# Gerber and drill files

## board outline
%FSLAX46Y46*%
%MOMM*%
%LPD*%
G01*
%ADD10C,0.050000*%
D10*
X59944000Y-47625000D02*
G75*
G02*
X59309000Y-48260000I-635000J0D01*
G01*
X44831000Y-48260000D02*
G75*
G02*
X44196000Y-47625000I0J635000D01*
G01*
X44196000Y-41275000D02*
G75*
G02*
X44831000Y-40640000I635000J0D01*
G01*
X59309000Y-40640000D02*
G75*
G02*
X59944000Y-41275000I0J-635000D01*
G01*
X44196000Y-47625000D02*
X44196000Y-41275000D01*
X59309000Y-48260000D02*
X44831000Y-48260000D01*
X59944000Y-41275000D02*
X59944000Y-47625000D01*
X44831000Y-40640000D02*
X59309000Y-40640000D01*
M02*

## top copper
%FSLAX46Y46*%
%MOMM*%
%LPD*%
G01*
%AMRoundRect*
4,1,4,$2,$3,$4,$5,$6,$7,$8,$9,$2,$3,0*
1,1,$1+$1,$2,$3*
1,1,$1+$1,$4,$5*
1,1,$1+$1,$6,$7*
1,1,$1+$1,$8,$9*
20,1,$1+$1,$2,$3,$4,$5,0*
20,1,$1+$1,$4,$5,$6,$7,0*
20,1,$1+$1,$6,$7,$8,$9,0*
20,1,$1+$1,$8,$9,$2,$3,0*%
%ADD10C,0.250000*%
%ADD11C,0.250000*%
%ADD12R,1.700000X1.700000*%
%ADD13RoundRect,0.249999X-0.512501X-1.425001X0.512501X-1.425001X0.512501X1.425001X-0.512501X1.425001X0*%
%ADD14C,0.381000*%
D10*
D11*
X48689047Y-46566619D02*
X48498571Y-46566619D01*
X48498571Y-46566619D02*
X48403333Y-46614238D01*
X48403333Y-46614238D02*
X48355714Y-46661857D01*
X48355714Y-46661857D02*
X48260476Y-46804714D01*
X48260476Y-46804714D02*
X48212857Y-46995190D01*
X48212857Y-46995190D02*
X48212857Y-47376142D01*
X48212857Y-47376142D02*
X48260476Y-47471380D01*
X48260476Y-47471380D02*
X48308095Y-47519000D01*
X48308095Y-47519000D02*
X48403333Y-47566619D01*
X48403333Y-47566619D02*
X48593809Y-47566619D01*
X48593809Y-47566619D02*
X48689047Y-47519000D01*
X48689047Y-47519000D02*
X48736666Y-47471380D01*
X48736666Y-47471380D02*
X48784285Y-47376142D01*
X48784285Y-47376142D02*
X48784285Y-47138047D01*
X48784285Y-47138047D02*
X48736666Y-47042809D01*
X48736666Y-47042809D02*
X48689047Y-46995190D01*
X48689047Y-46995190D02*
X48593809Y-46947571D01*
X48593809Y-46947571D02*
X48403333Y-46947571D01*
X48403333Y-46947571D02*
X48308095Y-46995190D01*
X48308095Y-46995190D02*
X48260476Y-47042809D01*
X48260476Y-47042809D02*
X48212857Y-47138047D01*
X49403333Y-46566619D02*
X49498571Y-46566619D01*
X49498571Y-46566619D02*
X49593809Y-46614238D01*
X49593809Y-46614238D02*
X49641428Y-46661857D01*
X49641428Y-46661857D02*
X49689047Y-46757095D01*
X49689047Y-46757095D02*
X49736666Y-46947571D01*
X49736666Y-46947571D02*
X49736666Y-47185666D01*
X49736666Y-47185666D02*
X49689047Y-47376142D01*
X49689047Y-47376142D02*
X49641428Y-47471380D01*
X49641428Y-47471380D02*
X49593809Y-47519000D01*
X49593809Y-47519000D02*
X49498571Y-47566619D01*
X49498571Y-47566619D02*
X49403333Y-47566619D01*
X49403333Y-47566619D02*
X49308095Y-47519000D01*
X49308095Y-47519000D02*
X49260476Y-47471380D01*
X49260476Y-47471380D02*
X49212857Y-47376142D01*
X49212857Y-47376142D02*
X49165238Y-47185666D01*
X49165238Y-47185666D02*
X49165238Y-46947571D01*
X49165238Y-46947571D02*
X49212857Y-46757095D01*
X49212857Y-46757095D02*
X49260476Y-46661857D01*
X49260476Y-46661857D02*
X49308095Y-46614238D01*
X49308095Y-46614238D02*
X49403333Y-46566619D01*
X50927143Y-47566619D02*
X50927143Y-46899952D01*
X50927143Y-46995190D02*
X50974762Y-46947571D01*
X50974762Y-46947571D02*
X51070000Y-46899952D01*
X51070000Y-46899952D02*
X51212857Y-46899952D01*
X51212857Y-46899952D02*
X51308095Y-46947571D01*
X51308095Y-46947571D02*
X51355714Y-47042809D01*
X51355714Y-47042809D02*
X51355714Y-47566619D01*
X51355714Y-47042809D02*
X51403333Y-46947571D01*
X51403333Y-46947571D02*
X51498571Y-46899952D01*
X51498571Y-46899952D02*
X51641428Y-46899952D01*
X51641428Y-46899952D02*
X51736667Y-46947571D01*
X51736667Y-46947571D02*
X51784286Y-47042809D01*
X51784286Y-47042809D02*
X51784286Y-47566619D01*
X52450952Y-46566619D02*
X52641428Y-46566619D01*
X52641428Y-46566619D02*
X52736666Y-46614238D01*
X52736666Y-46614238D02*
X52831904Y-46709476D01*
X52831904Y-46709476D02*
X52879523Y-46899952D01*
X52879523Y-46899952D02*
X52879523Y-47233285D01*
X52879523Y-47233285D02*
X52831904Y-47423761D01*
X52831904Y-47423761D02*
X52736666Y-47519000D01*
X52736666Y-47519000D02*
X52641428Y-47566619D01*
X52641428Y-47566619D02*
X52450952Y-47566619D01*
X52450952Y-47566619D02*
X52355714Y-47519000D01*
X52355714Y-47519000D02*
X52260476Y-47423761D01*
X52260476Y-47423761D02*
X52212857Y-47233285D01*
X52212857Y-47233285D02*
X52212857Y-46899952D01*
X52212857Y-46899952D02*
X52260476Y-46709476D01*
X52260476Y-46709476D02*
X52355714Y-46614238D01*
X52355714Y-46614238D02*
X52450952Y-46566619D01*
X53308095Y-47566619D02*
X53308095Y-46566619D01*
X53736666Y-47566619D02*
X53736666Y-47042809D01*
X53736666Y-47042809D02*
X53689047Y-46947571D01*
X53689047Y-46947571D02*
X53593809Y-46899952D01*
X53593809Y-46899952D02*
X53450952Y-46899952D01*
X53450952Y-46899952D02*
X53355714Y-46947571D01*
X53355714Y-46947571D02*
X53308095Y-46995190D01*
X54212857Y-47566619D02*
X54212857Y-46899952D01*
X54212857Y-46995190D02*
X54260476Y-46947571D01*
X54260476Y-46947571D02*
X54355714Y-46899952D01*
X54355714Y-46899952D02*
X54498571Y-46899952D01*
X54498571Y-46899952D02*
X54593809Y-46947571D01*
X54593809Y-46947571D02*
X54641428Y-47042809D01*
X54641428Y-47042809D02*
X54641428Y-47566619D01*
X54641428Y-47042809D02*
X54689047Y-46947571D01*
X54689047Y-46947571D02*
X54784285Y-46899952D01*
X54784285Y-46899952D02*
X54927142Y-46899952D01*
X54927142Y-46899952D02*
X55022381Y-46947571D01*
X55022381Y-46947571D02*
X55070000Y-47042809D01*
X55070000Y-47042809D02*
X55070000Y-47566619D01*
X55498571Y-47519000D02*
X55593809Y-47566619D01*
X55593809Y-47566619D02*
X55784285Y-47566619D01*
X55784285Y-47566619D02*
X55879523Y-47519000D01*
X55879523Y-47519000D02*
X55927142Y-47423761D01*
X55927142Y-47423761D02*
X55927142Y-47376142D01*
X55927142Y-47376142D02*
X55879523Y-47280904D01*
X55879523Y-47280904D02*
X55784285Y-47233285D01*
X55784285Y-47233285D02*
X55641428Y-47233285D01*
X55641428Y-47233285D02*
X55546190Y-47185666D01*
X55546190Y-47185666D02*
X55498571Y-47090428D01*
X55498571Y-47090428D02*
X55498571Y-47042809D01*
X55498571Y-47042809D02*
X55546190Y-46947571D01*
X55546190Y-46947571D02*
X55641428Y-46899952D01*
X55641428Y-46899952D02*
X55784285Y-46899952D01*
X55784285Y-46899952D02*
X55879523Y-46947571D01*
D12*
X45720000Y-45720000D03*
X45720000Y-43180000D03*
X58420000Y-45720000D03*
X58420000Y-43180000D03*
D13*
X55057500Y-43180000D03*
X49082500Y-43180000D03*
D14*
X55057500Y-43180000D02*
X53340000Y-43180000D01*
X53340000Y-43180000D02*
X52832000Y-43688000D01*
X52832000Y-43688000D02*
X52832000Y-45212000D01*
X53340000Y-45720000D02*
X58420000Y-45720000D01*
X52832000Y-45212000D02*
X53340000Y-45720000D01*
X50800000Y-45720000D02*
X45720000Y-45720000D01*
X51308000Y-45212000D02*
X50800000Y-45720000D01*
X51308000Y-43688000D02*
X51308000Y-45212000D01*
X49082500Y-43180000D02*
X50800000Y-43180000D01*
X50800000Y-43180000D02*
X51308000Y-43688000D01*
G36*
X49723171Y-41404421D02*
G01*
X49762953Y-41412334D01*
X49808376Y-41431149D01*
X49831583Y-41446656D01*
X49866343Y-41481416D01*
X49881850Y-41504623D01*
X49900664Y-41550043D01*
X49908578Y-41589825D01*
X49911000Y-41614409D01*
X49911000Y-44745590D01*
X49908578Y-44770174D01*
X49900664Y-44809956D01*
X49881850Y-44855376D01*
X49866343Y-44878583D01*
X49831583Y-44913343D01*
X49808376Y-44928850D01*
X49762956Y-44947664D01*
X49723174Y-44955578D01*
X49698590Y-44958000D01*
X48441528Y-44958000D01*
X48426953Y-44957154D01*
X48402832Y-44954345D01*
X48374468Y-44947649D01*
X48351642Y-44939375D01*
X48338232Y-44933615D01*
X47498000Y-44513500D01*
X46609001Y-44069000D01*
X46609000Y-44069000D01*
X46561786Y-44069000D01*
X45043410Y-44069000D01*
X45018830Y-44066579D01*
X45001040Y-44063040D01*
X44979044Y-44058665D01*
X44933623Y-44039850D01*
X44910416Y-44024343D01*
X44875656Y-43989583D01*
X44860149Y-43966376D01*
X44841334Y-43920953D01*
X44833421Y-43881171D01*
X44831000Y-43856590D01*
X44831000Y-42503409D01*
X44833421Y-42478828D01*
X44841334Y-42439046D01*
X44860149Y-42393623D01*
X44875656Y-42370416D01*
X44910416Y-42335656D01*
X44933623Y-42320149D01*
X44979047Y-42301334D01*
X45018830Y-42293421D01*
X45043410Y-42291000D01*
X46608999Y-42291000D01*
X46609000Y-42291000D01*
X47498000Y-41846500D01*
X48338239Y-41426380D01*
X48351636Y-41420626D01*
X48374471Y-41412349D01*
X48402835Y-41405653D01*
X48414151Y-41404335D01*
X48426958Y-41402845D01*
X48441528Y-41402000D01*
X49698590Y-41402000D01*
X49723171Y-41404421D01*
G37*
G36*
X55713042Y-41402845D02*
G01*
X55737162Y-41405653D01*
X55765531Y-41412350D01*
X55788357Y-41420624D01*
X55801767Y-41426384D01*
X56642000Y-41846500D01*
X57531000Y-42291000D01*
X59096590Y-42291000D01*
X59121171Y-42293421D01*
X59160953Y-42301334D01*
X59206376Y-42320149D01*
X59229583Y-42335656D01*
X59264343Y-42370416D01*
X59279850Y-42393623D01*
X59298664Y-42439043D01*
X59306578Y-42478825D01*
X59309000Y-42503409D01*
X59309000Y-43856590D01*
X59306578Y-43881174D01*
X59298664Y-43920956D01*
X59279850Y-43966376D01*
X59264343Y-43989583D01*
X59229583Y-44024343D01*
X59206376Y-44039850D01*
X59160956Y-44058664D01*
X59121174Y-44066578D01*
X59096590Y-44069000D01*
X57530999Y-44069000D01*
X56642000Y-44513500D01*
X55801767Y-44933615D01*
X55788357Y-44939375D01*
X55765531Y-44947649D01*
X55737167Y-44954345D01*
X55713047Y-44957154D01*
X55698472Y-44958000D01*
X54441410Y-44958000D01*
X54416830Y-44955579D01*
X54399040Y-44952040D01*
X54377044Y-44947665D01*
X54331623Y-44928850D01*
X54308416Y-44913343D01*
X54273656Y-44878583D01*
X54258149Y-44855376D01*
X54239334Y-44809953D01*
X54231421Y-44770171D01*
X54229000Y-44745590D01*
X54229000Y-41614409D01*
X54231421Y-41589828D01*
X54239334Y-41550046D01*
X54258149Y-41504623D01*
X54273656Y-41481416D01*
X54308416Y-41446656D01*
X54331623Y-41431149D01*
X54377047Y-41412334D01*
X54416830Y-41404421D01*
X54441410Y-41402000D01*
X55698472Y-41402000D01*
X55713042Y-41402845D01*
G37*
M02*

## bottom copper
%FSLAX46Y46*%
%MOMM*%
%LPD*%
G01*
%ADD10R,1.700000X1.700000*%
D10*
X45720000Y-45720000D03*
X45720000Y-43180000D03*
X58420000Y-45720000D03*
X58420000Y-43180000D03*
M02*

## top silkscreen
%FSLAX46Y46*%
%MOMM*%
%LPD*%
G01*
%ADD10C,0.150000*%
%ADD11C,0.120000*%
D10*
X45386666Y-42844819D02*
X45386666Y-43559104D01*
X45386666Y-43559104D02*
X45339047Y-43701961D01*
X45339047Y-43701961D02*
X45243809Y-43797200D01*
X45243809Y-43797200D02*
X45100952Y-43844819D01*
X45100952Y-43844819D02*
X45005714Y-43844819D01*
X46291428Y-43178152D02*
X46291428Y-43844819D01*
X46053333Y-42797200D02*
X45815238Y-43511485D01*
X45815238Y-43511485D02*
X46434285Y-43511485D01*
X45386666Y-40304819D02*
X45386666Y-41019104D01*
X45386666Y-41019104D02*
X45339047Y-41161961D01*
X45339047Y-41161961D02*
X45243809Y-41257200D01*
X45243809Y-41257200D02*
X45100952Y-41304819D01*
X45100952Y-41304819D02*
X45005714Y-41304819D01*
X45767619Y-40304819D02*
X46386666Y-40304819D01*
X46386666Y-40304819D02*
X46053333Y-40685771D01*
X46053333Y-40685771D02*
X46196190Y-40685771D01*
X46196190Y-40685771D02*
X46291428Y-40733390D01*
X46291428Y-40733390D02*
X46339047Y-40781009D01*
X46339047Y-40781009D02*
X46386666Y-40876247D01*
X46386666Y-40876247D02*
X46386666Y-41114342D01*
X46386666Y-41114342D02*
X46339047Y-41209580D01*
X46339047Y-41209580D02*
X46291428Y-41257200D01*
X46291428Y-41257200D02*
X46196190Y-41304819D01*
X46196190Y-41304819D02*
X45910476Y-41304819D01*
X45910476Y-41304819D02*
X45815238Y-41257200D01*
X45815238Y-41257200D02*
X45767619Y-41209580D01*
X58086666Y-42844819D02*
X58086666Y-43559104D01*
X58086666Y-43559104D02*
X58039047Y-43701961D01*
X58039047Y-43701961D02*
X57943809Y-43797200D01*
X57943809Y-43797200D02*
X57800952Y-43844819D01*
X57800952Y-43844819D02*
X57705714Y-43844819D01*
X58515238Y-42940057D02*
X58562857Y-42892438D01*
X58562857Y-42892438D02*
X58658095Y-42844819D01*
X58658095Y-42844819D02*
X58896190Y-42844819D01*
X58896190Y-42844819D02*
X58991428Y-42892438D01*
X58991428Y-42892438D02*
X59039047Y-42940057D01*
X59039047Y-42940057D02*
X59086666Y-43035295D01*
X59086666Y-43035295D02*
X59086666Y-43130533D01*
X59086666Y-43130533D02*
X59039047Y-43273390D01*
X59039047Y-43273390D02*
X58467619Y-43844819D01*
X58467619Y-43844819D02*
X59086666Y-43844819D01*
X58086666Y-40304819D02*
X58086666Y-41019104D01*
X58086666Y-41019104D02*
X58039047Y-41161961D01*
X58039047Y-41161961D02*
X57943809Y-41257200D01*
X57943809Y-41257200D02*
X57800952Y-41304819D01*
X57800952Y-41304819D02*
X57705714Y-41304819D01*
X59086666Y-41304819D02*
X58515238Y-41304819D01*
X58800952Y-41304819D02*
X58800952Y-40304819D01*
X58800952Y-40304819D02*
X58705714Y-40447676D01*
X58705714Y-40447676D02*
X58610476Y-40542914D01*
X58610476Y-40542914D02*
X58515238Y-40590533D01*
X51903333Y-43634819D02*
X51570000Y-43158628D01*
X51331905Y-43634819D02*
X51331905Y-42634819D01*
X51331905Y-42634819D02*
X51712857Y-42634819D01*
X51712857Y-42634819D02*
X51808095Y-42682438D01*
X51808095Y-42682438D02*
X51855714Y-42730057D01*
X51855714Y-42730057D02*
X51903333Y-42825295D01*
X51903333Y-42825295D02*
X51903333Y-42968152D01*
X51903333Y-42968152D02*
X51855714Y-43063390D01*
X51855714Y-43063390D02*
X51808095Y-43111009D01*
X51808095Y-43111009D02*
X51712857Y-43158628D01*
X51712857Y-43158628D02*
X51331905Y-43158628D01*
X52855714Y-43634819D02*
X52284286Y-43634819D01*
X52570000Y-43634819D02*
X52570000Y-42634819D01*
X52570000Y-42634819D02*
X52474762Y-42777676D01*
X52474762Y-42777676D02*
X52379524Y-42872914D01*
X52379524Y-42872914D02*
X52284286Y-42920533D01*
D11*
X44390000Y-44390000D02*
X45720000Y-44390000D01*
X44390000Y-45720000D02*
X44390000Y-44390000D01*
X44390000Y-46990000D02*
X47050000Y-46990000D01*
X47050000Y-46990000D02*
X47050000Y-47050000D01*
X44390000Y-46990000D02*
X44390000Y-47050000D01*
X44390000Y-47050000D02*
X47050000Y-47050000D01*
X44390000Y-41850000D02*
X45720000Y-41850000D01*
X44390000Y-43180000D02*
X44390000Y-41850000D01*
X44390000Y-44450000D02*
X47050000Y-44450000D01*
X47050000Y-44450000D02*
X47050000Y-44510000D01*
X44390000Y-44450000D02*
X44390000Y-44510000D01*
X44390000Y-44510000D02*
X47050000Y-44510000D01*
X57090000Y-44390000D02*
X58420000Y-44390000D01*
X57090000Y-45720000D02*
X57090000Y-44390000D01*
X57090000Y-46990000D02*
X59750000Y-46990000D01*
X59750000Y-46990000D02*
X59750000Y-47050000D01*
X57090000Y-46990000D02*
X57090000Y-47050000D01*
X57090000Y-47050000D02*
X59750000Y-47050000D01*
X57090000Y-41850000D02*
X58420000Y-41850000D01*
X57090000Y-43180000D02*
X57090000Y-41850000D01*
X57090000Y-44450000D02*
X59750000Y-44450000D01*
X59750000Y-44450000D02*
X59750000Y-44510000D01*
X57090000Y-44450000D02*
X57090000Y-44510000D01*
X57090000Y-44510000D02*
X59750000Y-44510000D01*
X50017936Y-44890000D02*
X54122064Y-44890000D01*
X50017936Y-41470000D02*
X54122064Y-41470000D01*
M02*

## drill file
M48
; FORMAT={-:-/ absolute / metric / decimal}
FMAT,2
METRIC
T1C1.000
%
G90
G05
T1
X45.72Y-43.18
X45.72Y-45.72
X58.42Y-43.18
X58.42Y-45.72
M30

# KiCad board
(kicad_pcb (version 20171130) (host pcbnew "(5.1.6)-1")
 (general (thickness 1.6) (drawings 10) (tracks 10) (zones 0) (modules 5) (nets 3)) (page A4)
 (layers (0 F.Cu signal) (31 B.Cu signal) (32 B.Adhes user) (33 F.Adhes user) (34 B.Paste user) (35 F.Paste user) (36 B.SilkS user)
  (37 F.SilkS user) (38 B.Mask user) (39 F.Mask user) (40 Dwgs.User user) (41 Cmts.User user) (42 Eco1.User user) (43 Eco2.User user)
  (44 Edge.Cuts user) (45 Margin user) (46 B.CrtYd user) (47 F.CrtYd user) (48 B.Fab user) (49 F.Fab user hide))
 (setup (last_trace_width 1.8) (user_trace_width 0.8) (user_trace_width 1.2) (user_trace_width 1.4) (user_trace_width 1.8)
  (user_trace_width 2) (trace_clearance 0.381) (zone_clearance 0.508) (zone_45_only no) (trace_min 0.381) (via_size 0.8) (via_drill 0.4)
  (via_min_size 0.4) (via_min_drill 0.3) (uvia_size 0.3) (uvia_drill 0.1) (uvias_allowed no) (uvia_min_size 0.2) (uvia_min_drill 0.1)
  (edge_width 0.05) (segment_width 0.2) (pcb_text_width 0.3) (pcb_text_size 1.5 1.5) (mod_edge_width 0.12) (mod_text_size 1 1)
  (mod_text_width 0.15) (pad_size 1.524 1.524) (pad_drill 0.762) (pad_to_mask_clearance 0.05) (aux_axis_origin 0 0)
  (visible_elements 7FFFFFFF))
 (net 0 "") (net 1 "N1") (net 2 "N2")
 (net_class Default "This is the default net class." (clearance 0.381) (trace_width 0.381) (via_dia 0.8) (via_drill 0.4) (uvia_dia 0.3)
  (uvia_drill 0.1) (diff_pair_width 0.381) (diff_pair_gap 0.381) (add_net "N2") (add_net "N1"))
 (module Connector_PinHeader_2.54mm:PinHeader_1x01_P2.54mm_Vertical (layer F.Cu) (at 45.72 45.72)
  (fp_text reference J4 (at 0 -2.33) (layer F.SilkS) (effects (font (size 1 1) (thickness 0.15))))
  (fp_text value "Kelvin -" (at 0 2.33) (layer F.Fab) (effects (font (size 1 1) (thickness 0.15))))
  (fp_line (start -1.33 -1.33) (end 0 -1.33) (layer F.SilkS) (width 0.12))
  (fp_line (start -1.33 0) (end -1.33 -1.33) (layer F.SilkS) (width 0.12))
  (fp_line (start -1.33 1.27) (end 1.33 1.27) (layer F.SilkS) (width 0.12))
  (fp_line (start 1.33 1.27) (end 1.33 1.33) (layer F.SilkS) (width 0.12))
  (fp_line (start -1.33 1.27) (end -1.33 1.33) (layer F.SilkS) (width 0.12))
  (fp_line (start -1.33 1.33) (end 1.33 1.33) (layer F.SilkS) (width 0.12))
  (pad 1 thru_hole rect (at 0 0) (size 1.7 1.7) (drill 1) (layers *.Cu *.Mask) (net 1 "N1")))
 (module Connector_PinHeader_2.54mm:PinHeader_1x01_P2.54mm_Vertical (layer F.Cu) (at 45.72 43.18)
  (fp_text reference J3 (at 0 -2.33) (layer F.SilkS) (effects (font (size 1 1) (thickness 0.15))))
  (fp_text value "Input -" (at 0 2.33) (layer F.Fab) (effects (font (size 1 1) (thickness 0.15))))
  (fp_line (start -1.33 -1.33) (end 0 -1.33) (layer F.SilkS) (width 0.12))
  (fp_line (start -1.33 0) (end -1.33 -1.33) (layer F.SilkS) (width 0.12))
  (fp_line (start -1.33 1.27) (end 1.33 1.27) (layer F.SilkS) (width 0.12))
  (fp_line (start 1.33 1.27) (end 1.33 1.33) (layer F.SilkS) (width 0.12))
  (fp_line (start -1.33 1.27) (end -1.33 1.33) (layer F.SilkS) (width 0.12))
  (fp_line (start -1.33 1.33) (end 1.33 1.33) (layer F.SilkS) (width 0.12))
  (pad 1 thru_hole rect (at 0 0) (size 1.7 1.7) (drill 1) (layers *.Cu *.Mask) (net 1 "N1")))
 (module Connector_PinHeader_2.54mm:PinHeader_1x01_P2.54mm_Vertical (layer F.Cu) (at 58.42 45.72)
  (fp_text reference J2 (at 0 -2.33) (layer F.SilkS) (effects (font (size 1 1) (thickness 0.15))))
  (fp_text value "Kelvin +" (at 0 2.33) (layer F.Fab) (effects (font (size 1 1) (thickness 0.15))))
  (fp_line (start -1.33 -1.33) (end 0 -1.33) (layer F.SilkS) (width 0.12))
  (fp_line (start -1.33 0) (end -1.33 -1.33) (layer F.SilkS) (width 0.12))
  (fp_line (start -1.33 1.27) (end 1.33 1.27) (layer F.SilkS) (width 0.12))
  (fp_line (start 1.33 1.27) (end 1.33 1.33) (layer F.SilkS) (width 0.12))
  (fp_line (start -1.33 1.27) (end -1.33 1.33) (layer F.SilkS) (width 0.12))
  (fp_line (start -1.33 1.33) (end 1.33 1.33) (layer F.SilkS) (width 0.12))
  (pad 1 thru_hole rect (at 0 0) (size 1.7 1.7) (drill 1) (layers *.Cu *.Mask) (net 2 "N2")))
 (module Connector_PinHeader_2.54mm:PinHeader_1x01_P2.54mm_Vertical (layer F.Cu) (at 58.42 43.18)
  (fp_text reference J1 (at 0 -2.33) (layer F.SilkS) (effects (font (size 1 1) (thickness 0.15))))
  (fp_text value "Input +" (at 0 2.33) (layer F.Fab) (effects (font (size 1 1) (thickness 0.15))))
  (fp_line (start -1.33 -1.33) (end 0 -1.33) (layer F.SilkS) (width 0.12))
  (fp_line (start -1.33 0) (end -1.33 -1.33) (layer F.SilkS) (width 0.12))
  (fp_line (start -1.33 1.27) (end 1.33 1.27) (layer F.SilkS) (width 0.12))
  (fp_line (start 1.33 1.27) (end 1.33 1.33) (layer F.SilkS) (width 0.12))
  (fp_line (start -1.33 1.27) (end -1.33 1.33) (layer F.SilkS) (width 0.12))
  (fp_line (start -1.33 1.33) (end 1.33 1.33) (layer F.SilkS) (width 0.12))
  (pad 1 thru_hole rect (at 0 0) (size 1.7 1.7) (drill 1) (layers *.Cu *.Mask) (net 2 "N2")))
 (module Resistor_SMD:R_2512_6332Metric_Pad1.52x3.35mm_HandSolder (layer F.Cu) (at 52.07 43.18)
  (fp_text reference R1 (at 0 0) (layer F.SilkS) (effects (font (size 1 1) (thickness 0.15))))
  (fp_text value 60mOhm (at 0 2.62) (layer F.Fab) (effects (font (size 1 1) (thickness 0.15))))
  (fp_line (start -2.052064 1.71) (end 2.052064 1.71) (layer F.SilkS) (width 0.12))
  (fp_line (start -2.052064 -1.71) (end 2.052064 -1.71) (layer F.SilkS) (width 0.12))
  (pad 2 smd roundrect (at 2.9875 0) (size 1.525 3.35) (layers F.Cu F.Paste F.Mask) (roundrect_rratio 0.163934) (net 2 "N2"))
  (pad 1 smd roundrect (at -2.9875 0) (size 1.525 3.35) (layers F.Cu F.Paste F.Mask) (roundrect_rratio 0.163934) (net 1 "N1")))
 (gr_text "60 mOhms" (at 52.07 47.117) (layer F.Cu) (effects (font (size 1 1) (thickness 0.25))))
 (gr_arc (start 59.309 47.625) (end 59.309 48.26) (angle -90) (layer Edge.Cuts) (width 0.05))
 (gr_arc (start 44.831 47.625) (end 44.196 47.625) (angle -90) (layer Edge.Cuts) (width 0.05))
 (gr_arc (start 44.831 41.275) (end 44.831 40.64) (angle -90) (layer Edge.Cuts) (width 0.05))
 (gr_arc (start 59.309 41.275) (end 59.944 41.275) (angle -90) (layer Edge.Cuts) (width 0.05))
 (gr_line (start 44.196 47.625) (end 44.196 41.275) (layer Edge.Cuts) (width 0.05))
 (gr_line (start 59.309 48.26) (end 44.831 48.26) (layer Edge.Cuts) (width 0.05))
 (gr_line (start 59.944 41.275) (end 59.944 47.625) (layer Edge.Cuts) (width 0.05))
 (gr_line (start 44.831 40.64) (end 59.309 40.64) (layer Edge.Cuts) (width 0.05))
 (segment (start 55.0575 43.18) (end 53.34 43.18) (width 0.381) (layer F.Cu) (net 2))
 (segment (start 53.34 43.18) (end 52.832 43.688) (width 0.381) (layer F.Cu) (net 2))
 (segment (start 52.832 43.688) (end 52.832 45.212) (width 0.381) (layer F.Cu) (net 2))
 (segment (start 53.34 45.72) (end 58.42 45.72) (width 0.381) (layer F.Cu) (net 2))
 (segment (start 52.832 45.212) (end 53.34 45.72) (width 0.381) (layer F.Cu) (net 2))
 (segment (start 50.8 45.72) (end 45.72 45.72) (width 0.381) (layer F.Cu) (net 1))
 (segment (start 51.308 45.212) (end 50.8 45.72) (width 0.381) (layer F.Cu) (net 1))
 (segment (start 51.308 43.688) (end 51.308 45.212) (width 0.381) (layer F.Cu) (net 1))
 (segment (start 49.0825 43.18) (end 50.8 43.18) (width 0.381) (layer F.Cu) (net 1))
 (segment (start 50.8 43.18) (end 51.308 43.688) (width 0.381) (layer F.Cu) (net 1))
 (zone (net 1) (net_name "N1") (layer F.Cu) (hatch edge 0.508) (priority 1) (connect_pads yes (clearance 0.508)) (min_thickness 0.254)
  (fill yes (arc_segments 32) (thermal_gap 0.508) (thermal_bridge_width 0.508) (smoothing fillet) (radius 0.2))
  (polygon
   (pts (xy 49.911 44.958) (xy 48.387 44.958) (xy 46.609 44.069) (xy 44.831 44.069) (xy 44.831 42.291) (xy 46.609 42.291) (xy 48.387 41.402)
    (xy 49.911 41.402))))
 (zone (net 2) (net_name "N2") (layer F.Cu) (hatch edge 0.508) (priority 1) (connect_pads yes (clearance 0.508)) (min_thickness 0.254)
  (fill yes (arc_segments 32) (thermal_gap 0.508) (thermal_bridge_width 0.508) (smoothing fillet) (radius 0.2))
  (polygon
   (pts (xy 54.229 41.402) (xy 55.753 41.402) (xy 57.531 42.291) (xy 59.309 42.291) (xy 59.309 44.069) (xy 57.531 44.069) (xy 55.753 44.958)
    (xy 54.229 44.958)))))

